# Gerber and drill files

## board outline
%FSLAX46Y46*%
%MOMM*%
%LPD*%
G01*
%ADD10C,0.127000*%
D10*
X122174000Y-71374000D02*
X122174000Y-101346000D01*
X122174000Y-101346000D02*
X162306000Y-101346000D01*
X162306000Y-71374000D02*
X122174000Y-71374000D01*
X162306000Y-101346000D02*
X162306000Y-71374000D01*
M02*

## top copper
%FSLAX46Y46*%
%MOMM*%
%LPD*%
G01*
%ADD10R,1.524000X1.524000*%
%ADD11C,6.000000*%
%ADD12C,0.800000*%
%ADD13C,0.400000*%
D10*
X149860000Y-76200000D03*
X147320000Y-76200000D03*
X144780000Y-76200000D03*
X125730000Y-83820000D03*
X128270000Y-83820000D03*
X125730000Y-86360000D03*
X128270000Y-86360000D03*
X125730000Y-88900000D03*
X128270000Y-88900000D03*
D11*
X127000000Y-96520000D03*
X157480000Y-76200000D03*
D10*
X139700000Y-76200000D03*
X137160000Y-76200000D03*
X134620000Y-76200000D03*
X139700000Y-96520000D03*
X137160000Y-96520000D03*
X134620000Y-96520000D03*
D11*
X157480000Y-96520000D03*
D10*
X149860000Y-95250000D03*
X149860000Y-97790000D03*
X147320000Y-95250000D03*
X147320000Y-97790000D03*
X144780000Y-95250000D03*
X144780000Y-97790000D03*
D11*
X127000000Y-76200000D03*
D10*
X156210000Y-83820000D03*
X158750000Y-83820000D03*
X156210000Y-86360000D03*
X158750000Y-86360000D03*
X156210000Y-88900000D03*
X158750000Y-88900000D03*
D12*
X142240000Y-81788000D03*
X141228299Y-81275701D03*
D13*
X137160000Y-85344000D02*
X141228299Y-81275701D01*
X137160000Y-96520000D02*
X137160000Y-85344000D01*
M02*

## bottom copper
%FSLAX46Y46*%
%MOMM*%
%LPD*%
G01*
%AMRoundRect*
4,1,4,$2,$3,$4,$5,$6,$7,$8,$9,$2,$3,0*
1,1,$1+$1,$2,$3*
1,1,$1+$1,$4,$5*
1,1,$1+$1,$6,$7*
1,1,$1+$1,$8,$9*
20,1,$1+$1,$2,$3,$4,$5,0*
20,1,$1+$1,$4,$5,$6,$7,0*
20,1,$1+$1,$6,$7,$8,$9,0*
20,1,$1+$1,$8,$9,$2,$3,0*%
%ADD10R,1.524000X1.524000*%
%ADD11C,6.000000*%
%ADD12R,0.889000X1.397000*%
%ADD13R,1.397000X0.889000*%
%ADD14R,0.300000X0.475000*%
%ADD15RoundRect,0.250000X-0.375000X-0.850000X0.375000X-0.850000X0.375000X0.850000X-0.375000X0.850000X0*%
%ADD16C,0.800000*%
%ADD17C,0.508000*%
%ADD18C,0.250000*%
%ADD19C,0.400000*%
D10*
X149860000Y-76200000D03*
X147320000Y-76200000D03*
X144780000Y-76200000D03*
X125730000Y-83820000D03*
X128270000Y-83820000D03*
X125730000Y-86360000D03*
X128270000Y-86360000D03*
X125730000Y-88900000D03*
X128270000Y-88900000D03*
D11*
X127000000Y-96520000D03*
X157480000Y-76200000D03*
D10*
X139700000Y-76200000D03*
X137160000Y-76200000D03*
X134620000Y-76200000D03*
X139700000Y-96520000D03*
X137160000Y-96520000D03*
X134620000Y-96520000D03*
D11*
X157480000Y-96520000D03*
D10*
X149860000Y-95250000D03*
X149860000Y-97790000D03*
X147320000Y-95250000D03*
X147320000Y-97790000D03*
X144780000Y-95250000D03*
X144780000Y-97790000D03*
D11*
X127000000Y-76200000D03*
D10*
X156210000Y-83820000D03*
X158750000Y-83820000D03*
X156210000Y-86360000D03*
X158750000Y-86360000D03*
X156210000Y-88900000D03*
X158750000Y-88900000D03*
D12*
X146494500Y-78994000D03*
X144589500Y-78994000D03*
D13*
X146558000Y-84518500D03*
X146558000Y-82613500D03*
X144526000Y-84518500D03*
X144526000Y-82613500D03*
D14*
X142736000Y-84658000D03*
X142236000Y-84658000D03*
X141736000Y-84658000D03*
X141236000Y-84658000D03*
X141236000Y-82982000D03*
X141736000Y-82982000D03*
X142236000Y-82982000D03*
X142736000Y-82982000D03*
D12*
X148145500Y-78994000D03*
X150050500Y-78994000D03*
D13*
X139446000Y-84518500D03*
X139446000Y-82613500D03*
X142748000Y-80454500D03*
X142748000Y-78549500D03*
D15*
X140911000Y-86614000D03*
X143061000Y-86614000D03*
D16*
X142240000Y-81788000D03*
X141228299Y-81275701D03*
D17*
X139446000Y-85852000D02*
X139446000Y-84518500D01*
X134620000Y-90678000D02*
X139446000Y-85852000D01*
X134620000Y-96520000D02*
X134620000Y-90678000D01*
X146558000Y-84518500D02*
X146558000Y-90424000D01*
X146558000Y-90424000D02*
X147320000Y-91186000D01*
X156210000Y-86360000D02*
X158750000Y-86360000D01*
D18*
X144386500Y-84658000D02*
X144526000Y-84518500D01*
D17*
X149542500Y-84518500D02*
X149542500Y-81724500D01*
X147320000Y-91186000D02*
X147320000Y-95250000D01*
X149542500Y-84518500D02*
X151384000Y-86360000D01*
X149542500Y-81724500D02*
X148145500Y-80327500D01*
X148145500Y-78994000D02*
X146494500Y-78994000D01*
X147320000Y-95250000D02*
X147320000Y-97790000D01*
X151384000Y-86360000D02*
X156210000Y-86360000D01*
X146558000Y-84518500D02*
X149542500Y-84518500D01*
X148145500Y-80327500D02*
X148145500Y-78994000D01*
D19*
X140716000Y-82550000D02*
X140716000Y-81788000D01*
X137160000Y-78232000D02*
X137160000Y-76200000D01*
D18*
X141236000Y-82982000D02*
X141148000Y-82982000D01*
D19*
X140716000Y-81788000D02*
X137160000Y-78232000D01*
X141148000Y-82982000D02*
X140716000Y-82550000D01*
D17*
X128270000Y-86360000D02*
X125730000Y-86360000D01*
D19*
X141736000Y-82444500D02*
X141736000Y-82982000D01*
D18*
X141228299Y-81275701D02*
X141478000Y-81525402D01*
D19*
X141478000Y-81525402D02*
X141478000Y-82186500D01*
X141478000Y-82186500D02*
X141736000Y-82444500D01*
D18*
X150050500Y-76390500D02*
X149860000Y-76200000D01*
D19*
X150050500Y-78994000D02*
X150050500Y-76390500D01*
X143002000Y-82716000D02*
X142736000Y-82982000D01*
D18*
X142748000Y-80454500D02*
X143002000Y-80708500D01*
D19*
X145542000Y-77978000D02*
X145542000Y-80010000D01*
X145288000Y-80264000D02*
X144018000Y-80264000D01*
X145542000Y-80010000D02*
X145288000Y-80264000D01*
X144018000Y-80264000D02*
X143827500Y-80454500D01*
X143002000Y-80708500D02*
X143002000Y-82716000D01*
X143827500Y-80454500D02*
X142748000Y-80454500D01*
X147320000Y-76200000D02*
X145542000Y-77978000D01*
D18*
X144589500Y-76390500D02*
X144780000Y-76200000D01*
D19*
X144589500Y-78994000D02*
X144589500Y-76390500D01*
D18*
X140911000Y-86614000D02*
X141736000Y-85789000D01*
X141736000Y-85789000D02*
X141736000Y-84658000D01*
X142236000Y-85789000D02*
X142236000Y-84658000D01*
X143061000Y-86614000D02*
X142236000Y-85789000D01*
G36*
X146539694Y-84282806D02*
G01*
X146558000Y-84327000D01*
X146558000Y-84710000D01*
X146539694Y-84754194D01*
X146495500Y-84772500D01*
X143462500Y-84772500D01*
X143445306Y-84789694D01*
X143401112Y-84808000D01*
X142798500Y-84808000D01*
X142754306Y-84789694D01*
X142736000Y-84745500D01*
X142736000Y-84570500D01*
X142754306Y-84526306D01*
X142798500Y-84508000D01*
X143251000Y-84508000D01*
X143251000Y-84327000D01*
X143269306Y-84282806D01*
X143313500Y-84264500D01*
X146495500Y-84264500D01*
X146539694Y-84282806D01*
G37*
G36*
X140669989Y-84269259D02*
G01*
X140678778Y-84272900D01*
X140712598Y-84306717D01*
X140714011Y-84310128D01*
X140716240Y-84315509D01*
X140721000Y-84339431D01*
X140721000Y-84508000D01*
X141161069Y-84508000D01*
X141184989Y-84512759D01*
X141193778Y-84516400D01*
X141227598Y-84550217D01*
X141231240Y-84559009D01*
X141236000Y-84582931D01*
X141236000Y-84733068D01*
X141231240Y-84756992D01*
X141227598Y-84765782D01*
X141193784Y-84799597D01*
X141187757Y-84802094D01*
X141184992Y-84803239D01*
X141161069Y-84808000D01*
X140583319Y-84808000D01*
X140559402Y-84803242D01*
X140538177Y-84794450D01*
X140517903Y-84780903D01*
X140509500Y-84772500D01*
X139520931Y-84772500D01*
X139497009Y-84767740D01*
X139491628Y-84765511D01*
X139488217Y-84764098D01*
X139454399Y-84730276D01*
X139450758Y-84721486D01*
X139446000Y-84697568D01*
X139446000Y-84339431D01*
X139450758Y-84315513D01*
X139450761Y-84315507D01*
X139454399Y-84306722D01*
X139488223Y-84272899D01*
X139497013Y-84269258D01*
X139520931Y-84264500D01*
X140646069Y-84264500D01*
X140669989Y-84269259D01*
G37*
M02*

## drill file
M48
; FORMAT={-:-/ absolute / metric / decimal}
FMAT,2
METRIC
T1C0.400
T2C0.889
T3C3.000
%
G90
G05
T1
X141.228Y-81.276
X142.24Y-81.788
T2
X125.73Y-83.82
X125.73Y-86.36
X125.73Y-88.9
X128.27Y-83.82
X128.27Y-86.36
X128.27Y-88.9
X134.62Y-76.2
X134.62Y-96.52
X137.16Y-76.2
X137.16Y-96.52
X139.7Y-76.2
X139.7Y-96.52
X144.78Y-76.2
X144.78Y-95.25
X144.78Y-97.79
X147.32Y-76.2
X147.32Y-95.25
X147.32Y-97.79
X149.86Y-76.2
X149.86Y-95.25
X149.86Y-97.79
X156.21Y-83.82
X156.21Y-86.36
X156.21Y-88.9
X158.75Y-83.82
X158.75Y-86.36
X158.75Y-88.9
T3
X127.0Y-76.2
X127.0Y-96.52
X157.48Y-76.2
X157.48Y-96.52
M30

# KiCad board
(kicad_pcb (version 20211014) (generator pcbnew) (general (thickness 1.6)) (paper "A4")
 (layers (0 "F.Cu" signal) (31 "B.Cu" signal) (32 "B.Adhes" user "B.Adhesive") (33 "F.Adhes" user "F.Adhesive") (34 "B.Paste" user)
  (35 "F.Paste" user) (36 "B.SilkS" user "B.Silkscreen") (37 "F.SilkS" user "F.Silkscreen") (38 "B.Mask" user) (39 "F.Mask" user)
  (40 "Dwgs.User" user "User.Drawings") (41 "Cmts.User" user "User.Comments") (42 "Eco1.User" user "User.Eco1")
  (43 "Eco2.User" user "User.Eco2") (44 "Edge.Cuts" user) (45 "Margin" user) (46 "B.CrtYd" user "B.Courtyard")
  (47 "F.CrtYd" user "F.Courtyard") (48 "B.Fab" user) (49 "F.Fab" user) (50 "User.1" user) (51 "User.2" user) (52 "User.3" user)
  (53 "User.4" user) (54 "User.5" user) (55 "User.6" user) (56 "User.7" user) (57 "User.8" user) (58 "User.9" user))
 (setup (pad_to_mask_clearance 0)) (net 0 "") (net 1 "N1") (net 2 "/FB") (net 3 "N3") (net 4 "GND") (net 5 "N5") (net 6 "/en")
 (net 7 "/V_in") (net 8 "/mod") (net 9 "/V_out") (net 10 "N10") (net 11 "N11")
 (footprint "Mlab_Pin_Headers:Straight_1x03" (layer "F.Cu") (at 147.32 76.2 -90)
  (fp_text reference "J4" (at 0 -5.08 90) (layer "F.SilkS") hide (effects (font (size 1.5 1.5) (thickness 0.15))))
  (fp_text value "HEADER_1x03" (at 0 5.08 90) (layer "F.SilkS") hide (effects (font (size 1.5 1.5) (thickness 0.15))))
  (pad "1" thru_hole rect (at 0 -2.54 270) (size 1.524 1.524) (drill 0.889) (layers *.Cu *.Mask) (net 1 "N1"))
  (pad "2" thru_hole rect (at 0 0 270) (size 1.524 1.524) (drill 0.889) (layers *.Cu *.Mask) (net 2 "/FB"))
  (pad "3" thru_hole rect (at 0 2.54 270) (size 1.524 1.524) (drill 0.889) (layers *.Cu *.Mask) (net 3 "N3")))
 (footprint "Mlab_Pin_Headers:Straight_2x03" (layer "F.Cu") (at 127 86.36)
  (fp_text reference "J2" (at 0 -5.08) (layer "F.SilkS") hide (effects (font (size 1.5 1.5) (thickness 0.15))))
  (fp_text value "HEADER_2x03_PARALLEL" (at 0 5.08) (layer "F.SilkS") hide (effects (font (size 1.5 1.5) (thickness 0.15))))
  (pad "1" thru_hole rect (at -1.27 -2.54) (size 1.524 1.524) (drill 0.889) (layers *.Cu *.Mask) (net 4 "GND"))
  (pad "2" thru_hole rect (at 1.27 -2.54) (size 1.524 1.524) (drill 0.889) (layers *.Cu *.Mask) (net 4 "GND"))
  (pad "3" thru_hole rect (at -1.27 0) (size 1.524 1.524) (drill 0.889) (layers *.Cu *.Mask) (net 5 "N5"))
  (pad "4" thru_hole rect (at 1.27 0) (size 1.524 1.524) (drill 0.889) (layers *.Cu *.Mask) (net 5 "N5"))
  (pad "5" thru_hole rect (at -1.27 2.54) (size 1.524 1.524) (drill 0.889) (layers *.Cu *.Mask) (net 4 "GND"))
  (pad "6" thru_hole rect (at 1.27 2.54) (size 1.524 1.524) (drill 0.889) (layers *.Cu *.Mask) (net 4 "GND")))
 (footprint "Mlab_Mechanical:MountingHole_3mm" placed (layer "F.Cu") (at 127 96.52)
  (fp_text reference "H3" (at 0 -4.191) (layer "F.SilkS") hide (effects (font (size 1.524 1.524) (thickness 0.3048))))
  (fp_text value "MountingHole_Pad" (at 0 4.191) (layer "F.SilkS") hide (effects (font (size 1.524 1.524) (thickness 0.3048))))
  (pad "1" thru_hole circle (at 0 0) (size 6 6) (drill 3) (layers *.Cu *.Mask) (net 4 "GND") (clearance 1) (zone_connect 2)))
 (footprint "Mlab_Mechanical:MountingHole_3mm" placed (layer "F.Cu") (at 157.48 76.2)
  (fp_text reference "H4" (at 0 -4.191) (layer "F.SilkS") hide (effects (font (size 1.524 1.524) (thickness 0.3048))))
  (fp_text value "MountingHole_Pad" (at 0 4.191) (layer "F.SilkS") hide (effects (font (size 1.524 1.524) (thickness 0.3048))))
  (pad "1" thru_hole circle (at 0 0) (size 6 6) (drill 3) (layers *.Cu *.Mask) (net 4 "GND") (clearance 1) (zone_connect 2)))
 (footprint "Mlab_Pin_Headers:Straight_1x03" (layer "F.Cu") (at 137.16 76.2 -90)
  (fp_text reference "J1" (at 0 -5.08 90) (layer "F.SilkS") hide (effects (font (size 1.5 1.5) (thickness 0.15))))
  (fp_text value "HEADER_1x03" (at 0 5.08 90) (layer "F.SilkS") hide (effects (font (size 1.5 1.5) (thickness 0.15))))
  (pad "1" thru_hole rect (at 0 -2.54 270) (size 1.524 1.524) (drill 0.889) (layers *.Cu *.Mask) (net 4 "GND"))
  (pad "2" thru_hole rect (at 0 0 270) (size 1.524 1.524) (drill 0.889) (layers *.Cu *.Mask) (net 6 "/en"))
  (pad "3" thru_hole rect (at 0 2.54 270) (size 1.524 1.524) (drill 0.889) (layers *.Cu *.Mask) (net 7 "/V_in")))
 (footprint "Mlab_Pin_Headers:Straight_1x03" (layer "F.Cu") (at 137.16 96.52 -90)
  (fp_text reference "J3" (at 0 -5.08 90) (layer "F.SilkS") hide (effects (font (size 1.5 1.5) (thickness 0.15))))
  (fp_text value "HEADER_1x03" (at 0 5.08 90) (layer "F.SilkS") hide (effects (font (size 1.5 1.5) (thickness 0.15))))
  (pad "1" thru_hole rect (at 0 -2.54 270) (size 1.524 1.524) (drill 0.889) (layers *.Cu *.Mask) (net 4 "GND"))
  (pad "2" thru_hole rect (at 0 0 270) (size 1.524 1.524) (drill 0.889) (layers *.Cu *.Mask) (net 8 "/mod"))
  (pad "3" thru_hole rect (at 0 2.54 270) (size 1.524 1.524) (drill 0.889) (layers *.Cu *.Mask) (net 7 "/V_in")))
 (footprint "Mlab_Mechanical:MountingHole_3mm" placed (layer "F.Cu") (at 157.48 96.52)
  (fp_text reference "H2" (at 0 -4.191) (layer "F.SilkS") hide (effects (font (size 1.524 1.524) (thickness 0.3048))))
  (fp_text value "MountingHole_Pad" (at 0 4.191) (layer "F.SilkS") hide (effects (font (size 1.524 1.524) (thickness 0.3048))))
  (pad "1" thru_hole circle (at 0 0) (size 6 6) (drill 3) (layers *.Cu *.Mask) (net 4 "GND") (clearance 1) (zone_connect 2)))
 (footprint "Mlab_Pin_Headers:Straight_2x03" (layer "F.Cu") (at 147.32 96.52 -90)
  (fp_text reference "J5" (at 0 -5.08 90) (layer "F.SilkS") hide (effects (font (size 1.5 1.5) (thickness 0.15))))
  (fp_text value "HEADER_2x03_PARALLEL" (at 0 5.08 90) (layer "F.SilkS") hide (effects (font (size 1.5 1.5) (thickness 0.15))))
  (pad "1" thru_hole rect (at -1.27 -2.54 270) (size 1.524 1.524) (drill 0.889) (layers *.Cu *.Mask) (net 4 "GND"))
  (pad "2" thru_hole rect (at 1.27 -2.54 270) (size 1.524 1.524) (drill 0.889) (layers *.Cu *.Mask) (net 4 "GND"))
  (pad "3" thru_hole rect (at -1.27 0 270) (size 1.524 1.524) (drill 0.889) (layers *.Cu *.Mask) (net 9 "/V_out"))
  (pad "4" thru_hole rect (at 1.27 0 270) (size 1.524 1.524) (drill 0.889) (layers *.Cu *.Mask) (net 9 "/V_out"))
  (pad "5" thru_hole rect (at -1.27 2.54 270) (size 1.524 1.524) (drill 0.889) (layers *.Cu *.Mask) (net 4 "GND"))
  (pad "6" thru_hole rect (at 1.27 2.54 270) (size 1.524 1.524) (drill 0.889) (layers *.Cu *.Mask) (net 4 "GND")))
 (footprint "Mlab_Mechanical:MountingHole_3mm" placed (layer "F.Cu") (at 127 76.2)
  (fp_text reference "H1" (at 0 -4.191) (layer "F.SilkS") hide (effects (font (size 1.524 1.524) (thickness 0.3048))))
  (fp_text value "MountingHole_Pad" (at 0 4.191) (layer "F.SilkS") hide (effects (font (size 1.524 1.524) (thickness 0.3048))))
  (pad "1" thru_hole circle (at 0 0) (size 6 6) (drill 3) (layers *.Cu *.Mask) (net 4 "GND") (clearance 1) (zone_connect 2)))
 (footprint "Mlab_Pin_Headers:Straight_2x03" (layer "F.Cu") (at 157.48 86.36)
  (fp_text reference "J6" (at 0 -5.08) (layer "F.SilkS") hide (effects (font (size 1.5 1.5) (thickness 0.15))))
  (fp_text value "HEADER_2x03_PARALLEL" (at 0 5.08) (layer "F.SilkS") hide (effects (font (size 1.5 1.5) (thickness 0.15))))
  (pad "1" thru_hole rect (at -1.27 -2.54) (size 1.524 1.524) (drill 0.889) (layers *.Cu *.Mask) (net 4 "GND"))
  (pad "2" thru_hole rect (at 1.27 -2.54) (size 1.524 1.524) (drill 0.889) (layers *.Cu *.Mask) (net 4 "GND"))
  (pad "3" thru_hole rect (at -1.27 0) (size 1.524 1.524) (drill 0.889) (layers *.Cu *.Mask) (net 9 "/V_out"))
  (pad "4" thru_hole rect (at 1.27 0) (size 1.524 1.524) (drill 0.889) (layers *.Cu *.Mask) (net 9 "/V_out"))
  (pad "5" thru_hole rect (at -1.27 2.54) (size 1.524 1.524) (drill 0.889) (layers *.Cu *.Mask) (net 4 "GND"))
  (pad "6" thru_hole rect (at 1.27 2.54) (size 1.524 1.524) (drill 0.889) (layers *.Cu *.Mask) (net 4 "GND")))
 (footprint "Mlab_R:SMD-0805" (layer "B.Cu") (at 145.542 78.994 180)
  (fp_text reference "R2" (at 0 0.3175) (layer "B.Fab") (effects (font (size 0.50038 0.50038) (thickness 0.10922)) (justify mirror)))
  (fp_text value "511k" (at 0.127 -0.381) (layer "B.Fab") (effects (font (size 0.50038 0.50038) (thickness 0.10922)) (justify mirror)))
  (pad "1" smd rect locked (at -0.9525 0 180) (size 0.889 1.397) (layers "B.Cu" "B.Paste" "B.Mask") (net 9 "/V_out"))
  (pad "2" smd rect locked (at 0.9525 0 180) (size 0.889 1.397) (layers "B.Cu" "B.Paste" "B.Mask") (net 3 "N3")))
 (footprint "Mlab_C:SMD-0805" (layer "B.Cu") (at 146.558 83.566 90)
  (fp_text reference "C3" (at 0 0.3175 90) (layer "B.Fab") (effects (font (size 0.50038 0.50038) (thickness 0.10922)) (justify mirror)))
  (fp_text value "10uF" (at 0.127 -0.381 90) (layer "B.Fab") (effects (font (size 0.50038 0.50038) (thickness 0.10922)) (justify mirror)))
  (pad "1" smd rect locked (at -0.9525 0 90) (size 0.889 1.397) (layers "B.Cu" "B.Paste" "B.Mask") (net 9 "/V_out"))
  (pad "2" smd rect locked (at 0.9525 0 90) (size 0.889 1.397) (layers "B.Cu" "B.Paste" "B.Mask") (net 4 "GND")))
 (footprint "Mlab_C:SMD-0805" (layer "B.Cu") (at 144.526 83.566 90)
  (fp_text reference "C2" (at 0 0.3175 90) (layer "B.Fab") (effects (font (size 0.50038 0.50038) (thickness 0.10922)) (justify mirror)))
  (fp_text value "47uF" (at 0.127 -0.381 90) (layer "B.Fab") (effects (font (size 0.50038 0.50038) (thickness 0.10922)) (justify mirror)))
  (pad "1" smd rect locked (at -0.9525 0 90) (size 0.889 1.397) (layers "B.Cu" "B.Paste" "B.Mask") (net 9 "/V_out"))
  (pad "2" smd rect locked (at 0.9525 0 90) (size 0.889 1.397) (layers "B.Cu" "B.Paste" "B.Mask") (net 4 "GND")))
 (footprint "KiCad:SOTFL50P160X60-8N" (layer "B.Cu") (at 141.986 83.82 90)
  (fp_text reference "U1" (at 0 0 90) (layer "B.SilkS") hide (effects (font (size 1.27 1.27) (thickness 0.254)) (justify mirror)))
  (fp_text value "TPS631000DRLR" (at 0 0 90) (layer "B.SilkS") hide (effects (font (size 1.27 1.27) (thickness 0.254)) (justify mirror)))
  (pad "1" smd rect locked (at -0.838 0.75) (size 0.3 0.475) (layers "B.Cu" "B.Paste" "B.Mask") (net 9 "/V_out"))
  (pad "2" smd rect locked (at -0.838 0.25) (size 0.3 0.475) (layers "B.Cu" "B.Paste" "B.Mask") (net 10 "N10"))
  (pad "3" smd rect locked (at -0.838 -0.25) (size 0.3 0.475) (layers "B.Cu" "B.Paste" "B.Mask") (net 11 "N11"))
  (pad "4" smd rect locked (at -0.838 -0.75) (size 0.3 0.475) (layers "B.Cu" "B.Paste" "B.Mask") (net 7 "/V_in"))
  (pad "5" smd rect locked (at 0.838 -0.75) (size 0.3 0.475) (layers "B.Cu" "B.Paste" "B.Mask") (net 6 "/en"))
  (pad "6" smd rect locked (at 0.838 -0.25) (size 0.3 0.475) (layers "B.Cu" "B.Paste" "B.Mask") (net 8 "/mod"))
  (pad "7" smd rect locked (at 0.838 0.25) (size 0.3 0.475) (layers "B.Cu" "B.Paste" "B.Mask") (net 4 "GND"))
  (pad "8" smd rect locked (at 0.838 0.75) (size 0.3 0.475) (layers "B.Cu" "B.Paste" "B.Mask") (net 2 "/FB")))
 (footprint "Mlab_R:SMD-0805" (layer "B.Cu") (at 149.098 78.994)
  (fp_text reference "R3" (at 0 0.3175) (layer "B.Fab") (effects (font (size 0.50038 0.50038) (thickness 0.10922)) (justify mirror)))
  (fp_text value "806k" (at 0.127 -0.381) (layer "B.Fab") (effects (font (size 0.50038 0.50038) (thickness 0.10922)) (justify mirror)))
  (pad "1" smd rect locked (at -0.9525 0) (size 0.889 1.397) (layers "B.Cu" "B.Paste" "B.Mask") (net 9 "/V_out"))
  (pad "2" smd rect locked (at 0.9525 0) (size 0.889 1.397) (layers "B.Cu" "B.Paste" "B.Mask") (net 1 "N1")))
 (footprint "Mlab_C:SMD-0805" (layer "B.Cu") (at 139.446 83.566 90)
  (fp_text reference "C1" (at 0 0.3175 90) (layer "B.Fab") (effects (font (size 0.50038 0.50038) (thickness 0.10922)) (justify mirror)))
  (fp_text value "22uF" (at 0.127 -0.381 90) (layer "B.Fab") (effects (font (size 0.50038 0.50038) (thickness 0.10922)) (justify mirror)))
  (pad "1" smd rect locked (at -0.9525 0 90) (size 0.889 1.397) (layers "B.Cu" "B.Paste" "B.Mask") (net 7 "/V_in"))
  (pad "2" smd rect locked (at 0.9525 0 90) (size 0.889 1.397) (layers "B.Cu" "B.Paste" "B.Mask") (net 4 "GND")))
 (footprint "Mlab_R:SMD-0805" (layer "B.Cu") (at 142.748 79.502 90)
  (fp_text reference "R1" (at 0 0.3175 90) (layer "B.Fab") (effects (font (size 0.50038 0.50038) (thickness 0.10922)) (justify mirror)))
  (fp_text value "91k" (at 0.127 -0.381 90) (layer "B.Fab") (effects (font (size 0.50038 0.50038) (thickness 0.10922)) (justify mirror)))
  (pad "1" smd rect locked (at -0.9525 0 90) (size 0.889 1.397) (layers "B.Cu" "B.Paste" "B.Mask") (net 2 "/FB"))
  (pad "2" smd rect locked (at 0.9525 0 90) (size 0.889 1.397) (layers "B.Cu" "B.Paste" "B.Mask") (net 4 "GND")))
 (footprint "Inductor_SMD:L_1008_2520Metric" (layer "B.Cu") (at 141.986 86.614)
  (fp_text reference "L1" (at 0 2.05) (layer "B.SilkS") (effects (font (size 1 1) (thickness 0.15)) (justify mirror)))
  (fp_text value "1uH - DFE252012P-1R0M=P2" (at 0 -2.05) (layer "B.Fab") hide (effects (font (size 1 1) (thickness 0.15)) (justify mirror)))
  (pad "1" smd roundrect (at -1.075 0) (size 1.25 2.2) (layers "B.Cu" "B.Paste" "B.Mask") (roundrect_rratio 0.2) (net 11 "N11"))
  (pad "2" smd roundrect (at 1.075 0) (size 1.25 2.2) (layers "B.Cu" "B.Paste" "B.Mask") (roundrect_rratio 0.2) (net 10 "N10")))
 (gr_line (start 122.174 71.374) (end 122.174 101.346) (layer "Edge.Cuts") (width 0.127))
 (gr_line (start 122.174 101.346) (end 162.306 101.346) (layer "Edge.Cuts") (width 0.127))
 (gr_line (start 162.306 71.374) (end 122.174 71.374) (layer "Edge.Cuts") (width 0.127))
 (gr_line (start 162.306 101.346) (end 162.306 71.374) (layer "Edge.Cuts") (width 0.127))
 (via (at 142.24 81.788) (size 0.8) (drill 0.4) (layers "F.Cu" "B.Cu") (free) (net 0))
 (segment (start 139.446 85.852) (end 139.446 84.5185) (width 0.508) (layer "B.Cu") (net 7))
 (segment (start 134.62 90.678) (end 139.446 85.852) (width 0.508) (layer "B.Cu") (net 7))
 (segment (start 134.62 96.52) (end 134.62 90.678) (width 0.508) (layer "B.Cu") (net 7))
 (segment (start 146.558 84.5185) (end 146.558 90.424) (width 0.508) (layer "B.Cu") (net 9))
 (segment (start 146.558 90.424) (end 147.32 91.186) (width 0.508) (layer "B.Cu") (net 9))
 (segment (start 156.21 86.36) (end 158.75 86.36) (width 0.508) (layer "B.Cu") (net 9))
 (segment (start 144.3865 84.658) (end 144.526 84.5185) (width 0.25) (layer "B.Cu") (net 9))
 (segment (start 149.5425 84.5185) (end 149.5425 81.7245) (width 0.508) (layer "B.Cu") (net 9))
 (segment (start 147.32 91.186) (end 147.32 95.25) (width 0.508) (layer "B.Cu") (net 9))
 (segment (start 149.5425 84.5185) (end 151.384 86.36) (width 0.508) (layer "B.Cu") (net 9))
 (segment (start 149.5425 81.7245) (end 148.1455 80.3275) (width 0.508) (layer "B.Cu") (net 9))
 (segment (start 148.1455 78.994) (end 146.4945 78.994) (width 0.508) (layer "B.Cu") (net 9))
 (segment (start 147.32 95.25) (end 147.32 97.79) (width 0.508) (layer "B.Cu") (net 9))
 (segment (start 151.384 86.36) (end 156.21 86.36) (width 0.508) (layer "B.Cu") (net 9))
 (segment (start 146.558 84.5185) (end 149.5425 84.5185) (width 0.508) (layer "B.Cu") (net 9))
 (segment (start 148.1455 80.3275) (end 148.1455 78.994) (width 0.508) (layer "B.Cu") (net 9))
 (segment (start 140.716 82.55) (end 140.716 81.788) (width 0.4) (layer "B.Cu") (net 6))
 (segment (start 137.16 78.232) (end 137.16 76.2) (width 0.4) (layer "B.Cu") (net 6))
 (segment (start 141.236 82.982) (end 141.148 82.982) (width 0.25) (layer "B.Cu") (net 6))
 (segment (start 140.716 81.788) (end 137.16 78.232) (width 0.4) (layer "B.Cu") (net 6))
 (segment (start 141.148 82.982) (end 140.716 82.55) (width 0.4) (layer "B.Cu") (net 6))
 (segment (start 128.27 86.36) (end 125.73 86.36) (width 0.508) (layer "B.Cu") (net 5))
 (segment (start 137.16 85.344) (end 141.228299 81.275701) (width 0.4) (layer "F.Cu") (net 8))
 (segment (start 137.16 96.52) (end 137.16 85.344) (width 0.4) (layer "F.Cu") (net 8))
 (via (at 141.228299 81.275701) (size 0.8) (drill 0.4) (layers "F.Cu" "B.Cu") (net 8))
 (segment (start 141.736 82.4445) (end 141.736 82.982) (width 0.4) (layer "B.Cu") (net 8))
 (segment (start 141.228299 81.275701) (end 141.478 81.525402) (width 0.25) (layer "B.Cu") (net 8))
 (segment (start 141.478 81.525402) (end 141.478 82.1865) (width 0.4) (layer "B.Cu") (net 8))
 (segment (start 141.478 82.1865) (end 141.736 82.4445) (width 0.4) (layer "B.Cu") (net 8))
 (segment (start 150.0505 76.3905) (end 149.86 76.2) (width 0.25) (layer "B.Cu") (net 1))
 (segment (start 150.0505 78.994) (end 150.0505 76.3905) (width 0.4) (layer "B.Cu") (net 1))
 (segment (start 143.002 82.716) (end 142.736 82.982) (width 0.4) (layer "B.Cu") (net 2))
 (segment (start 142.748 80.4545) (end 143.002 80.7085) (width 0.25) (layer "B.Cu") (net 2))
 (segment (start 145.542 77.978) (end 145.542 80.01) (width 0.4) (layer "B.Cu") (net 2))
 (segment (start 145.288 80.264) (end 144.018 80.264) (width 0.4) (layer "B.Cu") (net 2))
 (segment (start 145.542 80.01) (end 145.288 80.264) (width 0.4) (layer "B.Cu") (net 2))
 (segment (start 144.018 80.264) (end 143.8275 80.4545) (width 0.4) (layer "B.Cu") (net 2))
 (segment (start 143.002 80.7085) (end 143.002 82.716) (width 0.4) (layer "B.Cu") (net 2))
 (segment (start 143.8275 80.4545) (end 142.748 80.4545) (width 0.4) (layer "B.Cu") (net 2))
 (segment (start 147.32 76.2) (end 145.542 77.978) (width 0.4) (layer "B.Cu") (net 2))
 (segment (start 144.5895 76.3905) (end 144.78 76.2) (width 0.25) (layer "B.Cu") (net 3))
 (segment (start 144.5895 78.994) (end 144.5895 76.3905) (width 0.4) (layer "B.Cu") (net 3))
 (segment (start 140.911 86.614) (end 141.736 85.789) (width 0.25) (layer "B.Cu") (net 11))
 (segment (start 141.736 85.789) (end 141.736 84.658) (width 0.25) (layer "B.Cu") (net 11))
 (segment (start 142.236 85.789) (end 142.236 84.658) (width 0.25) (layer "B.Cu") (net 10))
 (segment (start 143.061 86.614) (end 142.236 85.789) (width 0.25) (layer "B.Cu") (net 10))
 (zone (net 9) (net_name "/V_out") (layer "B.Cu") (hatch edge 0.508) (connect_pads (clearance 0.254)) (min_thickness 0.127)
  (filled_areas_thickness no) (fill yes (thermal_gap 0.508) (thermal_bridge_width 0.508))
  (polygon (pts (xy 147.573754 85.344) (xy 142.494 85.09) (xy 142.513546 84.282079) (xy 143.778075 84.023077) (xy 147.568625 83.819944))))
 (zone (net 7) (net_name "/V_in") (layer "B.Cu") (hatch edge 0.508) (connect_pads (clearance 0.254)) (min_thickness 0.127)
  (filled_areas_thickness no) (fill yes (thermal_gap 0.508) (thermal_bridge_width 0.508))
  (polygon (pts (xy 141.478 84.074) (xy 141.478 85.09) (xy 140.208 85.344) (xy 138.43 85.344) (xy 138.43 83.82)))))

